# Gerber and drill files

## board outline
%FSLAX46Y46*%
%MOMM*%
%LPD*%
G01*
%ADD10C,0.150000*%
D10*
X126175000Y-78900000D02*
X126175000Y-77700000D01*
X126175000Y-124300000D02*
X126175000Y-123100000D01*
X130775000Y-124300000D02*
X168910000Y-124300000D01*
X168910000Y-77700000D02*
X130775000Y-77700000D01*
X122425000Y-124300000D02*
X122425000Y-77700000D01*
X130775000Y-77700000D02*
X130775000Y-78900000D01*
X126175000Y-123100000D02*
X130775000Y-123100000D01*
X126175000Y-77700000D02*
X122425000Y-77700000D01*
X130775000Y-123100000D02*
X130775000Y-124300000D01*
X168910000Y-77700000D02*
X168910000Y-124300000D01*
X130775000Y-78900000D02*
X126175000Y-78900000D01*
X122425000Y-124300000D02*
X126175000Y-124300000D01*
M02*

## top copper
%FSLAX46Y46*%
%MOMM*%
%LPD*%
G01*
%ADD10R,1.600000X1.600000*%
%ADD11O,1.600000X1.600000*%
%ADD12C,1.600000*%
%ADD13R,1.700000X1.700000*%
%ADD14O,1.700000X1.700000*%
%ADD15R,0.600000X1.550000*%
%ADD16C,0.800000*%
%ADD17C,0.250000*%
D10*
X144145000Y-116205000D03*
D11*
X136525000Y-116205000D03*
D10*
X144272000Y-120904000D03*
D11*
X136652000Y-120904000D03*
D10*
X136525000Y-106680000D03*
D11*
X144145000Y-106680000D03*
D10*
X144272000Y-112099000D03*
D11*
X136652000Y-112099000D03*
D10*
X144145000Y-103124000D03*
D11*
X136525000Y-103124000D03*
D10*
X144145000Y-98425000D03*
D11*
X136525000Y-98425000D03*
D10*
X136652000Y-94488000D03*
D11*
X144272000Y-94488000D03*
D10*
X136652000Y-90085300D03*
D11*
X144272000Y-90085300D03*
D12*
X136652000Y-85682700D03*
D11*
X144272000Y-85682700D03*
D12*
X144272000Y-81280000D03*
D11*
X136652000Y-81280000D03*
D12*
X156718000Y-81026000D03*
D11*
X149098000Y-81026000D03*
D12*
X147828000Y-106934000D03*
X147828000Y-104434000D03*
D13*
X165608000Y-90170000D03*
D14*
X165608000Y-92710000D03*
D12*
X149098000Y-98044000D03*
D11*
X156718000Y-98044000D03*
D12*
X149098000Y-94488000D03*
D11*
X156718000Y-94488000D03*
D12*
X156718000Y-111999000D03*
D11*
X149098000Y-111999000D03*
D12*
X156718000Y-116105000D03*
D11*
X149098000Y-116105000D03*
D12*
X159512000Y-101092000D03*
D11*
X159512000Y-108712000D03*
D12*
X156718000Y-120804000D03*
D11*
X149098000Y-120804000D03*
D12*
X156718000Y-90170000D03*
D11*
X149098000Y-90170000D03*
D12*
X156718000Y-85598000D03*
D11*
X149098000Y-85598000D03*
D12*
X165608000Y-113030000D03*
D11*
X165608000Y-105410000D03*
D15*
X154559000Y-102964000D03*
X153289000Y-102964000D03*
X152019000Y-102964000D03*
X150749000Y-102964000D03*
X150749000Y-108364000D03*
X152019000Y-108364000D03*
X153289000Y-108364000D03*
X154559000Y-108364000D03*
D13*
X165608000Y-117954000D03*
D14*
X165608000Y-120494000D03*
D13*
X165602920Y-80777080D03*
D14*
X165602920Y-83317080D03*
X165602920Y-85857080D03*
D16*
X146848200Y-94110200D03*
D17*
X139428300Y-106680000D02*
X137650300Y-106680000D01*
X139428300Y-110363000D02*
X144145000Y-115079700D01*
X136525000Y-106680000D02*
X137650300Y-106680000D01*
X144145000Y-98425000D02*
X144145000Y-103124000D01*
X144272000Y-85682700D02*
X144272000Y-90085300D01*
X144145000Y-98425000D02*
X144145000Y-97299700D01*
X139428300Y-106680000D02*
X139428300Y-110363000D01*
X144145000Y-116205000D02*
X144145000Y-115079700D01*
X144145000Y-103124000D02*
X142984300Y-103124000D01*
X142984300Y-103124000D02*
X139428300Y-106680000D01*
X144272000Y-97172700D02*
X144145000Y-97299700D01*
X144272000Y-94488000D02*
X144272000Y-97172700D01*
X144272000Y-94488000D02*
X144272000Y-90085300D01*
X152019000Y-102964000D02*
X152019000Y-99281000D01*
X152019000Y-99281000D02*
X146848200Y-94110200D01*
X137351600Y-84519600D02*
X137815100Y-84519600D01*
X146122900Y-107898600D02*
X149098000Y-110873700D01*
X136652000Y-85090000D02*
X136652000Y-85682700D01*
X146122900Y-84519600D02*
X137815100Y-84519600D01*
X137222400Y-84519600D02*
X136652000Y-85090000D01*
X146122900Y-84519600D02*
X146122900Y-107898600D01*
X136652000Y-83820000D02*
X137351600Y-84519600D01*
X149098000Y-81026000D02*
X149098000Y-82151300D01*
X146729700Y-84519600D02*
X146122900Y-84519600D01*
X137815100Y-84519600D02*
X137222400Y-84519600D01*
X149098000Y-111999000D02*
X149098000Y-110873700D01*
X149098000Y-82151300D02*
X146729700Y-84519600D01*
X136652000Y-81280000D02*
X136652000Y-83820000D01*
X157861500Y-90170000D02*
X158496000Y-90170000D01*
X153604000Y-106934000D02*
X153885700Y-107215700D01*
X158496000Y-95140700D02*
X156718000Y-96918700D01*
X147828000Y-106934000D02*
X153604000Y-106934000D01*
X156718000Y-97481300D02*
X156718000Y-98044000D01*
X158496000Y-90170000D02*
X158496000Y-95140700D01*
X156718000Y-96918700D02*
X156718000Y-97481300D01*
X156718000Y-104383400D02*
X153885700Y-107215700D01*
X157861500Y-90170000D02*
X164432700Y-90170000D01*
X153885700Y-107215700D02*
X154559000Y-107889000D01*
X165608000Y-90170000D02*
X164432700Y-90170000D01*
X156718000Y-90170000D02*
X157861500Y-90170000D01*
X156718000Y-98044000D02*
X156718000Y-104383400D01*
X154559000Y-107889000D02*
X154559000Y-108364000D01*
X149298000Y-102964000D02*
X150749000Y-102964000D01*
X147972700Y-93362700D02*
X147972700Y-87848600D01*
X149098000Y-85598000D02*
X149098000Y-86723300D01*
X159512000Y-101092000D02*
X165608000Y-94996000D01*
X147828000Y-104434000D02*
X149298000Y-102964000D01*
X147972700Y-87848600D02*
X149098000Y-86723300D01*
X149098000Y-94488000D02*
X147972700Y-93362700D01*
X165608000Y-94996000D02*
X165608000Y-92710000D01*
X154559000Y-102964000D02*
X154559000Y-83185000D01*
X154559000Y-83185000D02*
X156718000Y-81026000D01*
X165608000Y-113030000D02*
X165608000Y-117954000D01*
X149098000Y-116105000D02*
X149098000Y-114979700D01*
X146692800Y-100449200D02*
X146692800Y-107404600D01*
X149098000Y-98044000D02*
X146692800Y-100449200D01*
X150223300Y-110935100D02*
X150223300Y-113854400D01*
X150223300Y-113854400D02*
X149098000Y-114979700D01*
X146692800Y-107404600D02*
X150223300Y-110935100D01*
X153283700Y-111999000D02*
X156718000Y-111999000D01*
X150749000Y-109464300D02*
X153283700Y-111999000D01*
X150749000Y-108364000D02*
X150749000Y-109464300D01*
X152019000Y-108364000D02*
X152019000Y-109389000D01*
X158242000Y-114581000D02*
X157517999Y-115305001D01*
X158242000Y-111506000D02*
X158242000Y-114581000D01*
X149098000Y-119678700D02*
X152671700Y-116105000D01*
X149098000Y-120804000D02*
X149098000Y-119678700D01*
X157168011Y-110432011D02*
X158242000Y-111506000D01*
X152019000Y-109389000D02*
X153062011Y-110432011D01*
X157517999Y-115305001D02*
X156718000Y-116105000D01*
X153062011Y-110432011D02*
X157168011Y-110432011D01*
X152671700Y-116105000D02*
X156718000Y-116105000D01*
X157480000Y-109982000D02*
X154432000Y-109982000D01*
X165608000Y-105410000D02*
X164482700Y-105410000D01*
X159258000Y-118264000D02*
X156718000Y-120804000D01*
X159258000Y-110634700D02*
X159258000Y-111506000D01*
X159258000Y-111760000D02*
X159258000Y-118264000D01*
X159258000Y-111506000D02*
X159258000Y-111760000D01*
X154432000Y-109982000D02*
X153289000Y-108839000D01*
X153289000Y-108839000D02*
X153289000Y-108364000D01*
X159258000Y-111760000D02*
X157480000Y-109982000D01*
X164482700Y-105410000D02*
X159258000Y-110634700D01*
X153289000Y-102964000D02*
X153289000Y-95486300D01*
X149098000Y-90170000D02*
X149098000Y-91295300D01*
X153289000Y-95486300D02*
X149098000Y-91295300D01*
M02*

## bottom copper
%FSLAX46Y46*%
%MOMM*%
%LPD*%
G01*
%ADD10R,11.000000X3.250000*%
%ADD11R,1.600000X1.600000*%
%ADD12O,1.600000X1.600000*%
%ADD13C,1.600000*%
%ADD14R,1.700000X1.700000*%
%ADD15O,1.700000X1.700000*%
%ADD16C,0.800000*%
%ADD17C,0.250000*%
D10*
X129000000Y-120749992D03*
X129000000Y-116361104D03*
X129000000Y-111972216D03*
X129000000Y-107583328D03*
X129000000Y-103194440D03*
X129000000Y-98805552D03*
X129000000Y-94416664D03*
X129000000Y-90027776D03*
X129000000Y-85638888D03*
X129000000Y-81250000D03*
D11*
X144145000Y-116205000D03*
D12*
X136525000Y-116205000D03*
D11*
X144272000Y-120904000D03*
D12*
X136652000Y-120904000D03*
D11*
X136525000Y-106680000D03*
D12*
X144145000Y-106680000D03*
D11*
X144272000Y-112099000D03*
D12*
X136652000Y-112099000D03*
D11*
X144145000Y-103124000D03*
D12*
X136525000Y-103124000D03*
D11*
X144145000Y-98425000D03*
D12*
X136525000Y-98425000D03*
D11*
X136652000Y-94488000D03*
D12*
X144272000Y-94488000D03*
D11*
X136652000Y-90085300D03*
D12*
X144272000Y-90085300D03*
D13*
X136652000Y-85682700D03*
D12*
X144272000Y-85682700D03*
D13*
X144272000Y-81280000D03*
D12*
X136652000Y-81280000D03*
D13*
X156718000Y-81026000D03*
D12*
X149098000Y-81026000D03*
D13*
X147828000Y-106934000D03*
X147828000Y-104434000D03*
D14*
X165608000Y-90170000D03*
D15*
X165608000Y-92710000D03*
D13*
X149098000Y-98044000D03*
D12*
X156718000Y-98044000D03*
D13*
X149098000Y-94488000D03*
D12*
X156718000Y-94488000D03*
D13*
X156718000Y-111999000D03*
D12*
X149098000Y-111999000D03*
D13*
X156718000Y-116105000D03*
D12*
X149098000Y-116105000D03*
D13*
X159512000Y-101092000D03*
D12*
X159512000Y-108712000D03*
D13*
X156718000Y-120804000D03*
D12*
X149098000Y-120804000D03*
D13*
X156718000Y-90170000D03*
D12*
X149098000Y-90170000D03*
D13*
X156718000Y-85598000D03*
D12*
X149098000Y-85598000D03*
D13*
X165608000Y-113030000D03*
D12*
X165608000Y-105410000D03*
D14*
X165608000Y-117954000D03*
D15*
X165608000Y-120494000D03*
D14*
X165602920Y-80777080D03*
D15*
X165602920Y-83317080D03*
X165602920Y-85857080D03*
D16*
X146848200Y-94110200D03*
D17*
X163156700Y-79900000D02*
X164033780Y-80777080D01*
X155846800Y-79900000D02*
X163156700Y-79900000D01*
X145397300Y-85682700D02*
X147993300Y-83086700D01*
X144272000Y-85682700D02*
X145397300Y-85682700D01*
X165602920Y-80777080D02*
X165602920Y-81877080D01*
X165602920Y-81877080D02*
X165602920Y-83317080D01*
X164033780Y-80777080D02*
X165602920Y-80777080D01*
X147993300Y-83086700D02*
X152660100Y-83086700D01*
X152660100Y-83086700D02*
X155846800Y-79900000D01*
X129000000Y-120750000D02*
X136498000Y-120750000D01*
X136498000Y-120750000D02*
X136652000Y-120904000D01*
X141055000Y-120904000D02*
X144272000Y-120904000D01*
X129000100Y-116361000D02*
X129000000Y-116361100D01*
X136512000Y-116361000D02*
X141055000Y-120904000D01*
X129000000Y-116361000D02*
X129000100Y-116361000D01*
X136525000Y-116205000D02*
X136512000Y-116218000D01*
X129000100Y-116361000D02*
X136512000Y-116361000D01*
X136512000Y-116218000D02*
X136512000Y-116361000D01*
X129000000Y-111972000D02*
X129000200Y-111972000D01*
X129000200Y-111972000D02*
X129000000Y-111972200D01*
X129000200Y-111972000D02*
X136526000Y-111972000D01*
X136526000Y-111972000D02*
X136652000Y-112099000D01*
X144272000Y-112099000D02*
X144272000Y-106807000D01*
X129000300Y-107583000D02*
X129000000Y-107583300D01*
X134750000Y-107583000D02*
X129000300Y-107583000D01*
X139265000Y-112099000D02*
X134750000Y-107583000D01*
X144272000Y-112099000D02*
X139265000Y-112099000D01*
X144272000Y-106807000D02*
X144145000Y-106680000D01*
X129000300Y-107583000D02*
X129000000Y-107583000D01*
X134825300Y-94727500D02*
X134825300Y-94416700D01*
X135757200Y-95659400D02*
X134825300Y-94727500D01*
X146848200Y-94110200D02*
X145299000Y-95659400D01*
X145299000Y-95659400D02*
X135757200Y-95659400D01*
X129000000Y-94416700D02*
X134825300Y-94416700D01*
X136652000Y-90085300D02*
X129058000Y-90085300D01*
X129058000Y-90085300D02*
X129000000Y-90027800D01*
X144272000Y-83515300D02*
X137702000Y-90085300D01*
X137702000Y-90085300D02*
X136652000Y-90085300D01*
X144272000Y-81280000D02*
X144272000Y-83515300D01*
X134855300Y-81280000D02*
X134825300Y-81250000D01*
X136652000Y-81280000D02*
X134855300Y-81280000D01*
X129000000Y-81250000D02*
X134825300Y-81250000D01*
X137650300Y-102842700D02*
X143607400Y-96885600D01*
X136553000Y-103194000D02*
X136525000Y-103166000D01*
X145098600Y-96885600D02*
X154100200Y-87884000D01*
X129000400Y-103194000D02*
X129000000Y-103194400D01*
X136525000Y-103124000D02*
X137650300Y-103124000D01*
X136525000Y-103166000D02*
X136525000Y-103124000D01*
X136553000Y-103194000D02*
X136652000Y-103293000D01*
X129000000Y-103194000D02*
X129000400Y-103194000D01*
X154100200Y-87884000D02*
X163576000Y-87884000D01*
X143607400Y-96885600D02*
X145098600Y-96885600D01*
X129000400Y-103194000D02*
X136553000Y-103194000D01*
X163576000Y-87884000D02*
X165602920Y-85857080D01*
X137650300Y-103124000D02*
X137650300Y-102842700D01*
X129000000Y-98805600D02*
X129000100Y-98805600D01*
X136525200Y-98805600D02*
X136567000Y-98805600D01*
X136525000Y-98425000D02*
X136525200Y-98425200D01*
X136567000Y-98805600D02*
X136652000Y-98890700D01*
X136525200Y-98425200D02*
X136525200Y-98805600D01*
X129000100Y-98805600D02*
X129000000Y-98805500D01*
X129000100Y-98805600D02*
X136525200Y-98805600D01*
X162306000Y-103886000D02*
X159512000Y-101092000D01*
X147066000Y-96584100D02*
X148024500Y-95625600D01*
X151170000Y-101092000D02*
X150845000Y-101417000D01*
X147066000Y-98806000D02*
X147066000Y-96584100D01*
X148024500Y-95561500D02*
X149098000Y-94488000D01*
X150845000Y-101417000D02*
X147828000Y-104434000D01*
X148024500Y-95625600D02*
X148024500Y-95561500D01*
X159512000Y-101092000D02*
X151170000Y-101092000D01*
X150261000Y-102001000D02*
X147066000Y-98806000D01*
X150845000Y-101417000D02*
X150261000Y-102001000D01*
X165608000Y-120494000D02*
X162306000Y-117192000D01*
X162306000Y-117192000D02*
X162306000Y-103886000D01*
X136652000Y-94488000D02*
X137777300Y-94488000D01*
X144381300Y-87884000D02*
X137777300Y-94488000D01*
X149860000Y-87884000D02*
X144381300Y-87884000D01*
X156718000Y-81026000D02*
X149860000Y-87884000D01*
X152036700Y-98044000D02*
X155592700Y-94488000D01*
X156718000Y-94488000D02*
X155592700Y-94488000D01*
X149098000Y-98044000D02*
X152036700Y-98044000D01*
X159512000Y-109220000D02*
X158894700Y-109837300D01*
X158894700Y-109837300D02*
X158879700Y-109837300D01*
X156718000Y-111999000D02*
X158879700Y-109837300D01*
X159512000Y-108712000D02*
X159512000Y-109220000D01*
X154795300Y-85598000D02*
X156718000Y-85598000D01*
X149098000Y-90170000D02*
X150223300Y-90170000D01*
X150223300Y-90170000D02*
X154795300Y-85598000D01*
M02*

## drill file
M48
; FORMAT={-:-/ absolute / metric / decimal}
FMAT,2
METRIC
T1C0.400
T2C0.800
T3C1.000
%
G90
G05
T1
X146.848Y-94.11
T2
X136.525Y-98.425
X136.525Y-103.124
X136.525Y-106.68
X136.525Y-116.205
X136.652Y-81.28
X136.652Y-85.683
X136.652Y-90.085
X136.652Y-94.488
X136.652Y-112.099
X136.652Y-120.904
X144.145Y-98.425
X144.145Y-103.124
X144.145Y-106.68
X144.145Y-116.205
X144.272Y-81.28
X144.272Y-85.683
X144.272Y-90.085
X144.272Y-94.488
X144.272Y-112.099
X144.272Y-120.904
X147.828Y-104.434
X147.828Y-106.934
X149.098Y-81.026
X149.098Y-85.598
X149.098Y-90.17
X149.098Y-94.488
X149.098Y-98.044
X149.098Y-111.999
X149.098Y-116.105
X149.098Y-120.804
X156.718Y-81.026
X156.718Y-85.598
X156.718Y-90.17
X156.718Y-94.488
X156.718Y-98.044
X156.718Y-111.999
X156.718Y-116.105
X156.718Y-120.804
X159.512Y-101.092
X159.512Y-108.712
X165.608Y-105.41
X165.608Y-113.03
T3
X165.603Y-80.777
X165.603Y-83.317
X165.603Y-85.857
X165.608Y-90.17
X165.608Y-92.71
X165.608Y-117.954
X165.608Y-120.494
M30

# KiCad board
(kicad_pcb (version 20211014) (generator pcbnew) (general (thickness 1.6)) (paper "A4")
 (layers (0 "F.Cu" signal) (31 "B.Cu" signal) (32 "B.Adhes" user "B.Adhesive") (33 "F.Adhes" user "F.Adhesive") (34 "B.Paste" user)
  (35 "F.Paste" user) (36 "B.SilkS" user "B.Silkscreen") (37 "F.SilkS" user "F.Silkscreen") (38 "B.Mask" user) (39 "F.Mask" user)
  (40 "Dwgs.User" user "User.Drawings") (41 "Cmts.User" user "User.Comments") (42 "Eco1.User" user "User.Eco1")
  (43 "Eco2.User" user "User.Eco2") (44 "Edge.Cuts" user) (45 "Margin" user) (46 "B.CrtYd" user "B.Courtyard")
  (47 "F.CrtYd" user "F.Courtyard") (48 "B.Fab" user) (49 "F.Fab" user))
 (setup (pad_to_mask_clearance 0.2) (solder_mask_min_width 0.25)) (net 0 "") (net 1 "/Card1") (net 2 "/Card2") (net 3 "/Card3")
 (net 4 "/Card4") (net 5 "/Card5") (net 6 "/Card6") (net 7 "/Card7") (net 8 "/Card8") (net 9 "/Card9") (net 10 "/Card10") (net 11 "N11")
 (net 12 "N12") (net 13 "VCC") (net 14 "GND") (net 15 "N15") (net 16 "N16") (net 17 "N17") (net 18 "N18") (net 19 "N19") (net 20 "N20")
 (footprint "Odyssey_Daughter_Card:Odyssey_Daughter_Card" (layer "F.Cu") (at 129 101)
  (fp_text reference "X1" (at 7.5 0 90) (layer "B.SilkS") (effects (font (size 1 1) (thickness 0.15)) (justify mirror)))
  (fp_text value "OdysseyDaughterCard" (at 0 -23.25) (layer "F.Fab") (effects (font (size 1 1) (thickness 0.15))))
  (pad "1" smd rect locked (at 0 19.749992) (size 11 3.25) (layers "B.Cu" "B.Mask") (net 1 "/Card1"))
  (pad "2" smd rect locked (at 0 15.361104) (size 11 3.25) (layers "B.Cu" "B.Mask") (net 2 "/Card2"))
  (pad "3" smd rect locked (at 0 10.972216) (size 11 3.25) (layers "B.Cu" "B.Mask") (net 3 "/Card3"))
  (pad "4" smd rect locked (at 0 6.583328) (size 11 3.25) (layers "B.Cu" "B.Mask") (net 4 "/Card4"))
  (pad "5" smd rect locked (at 0 2.19444) (size 11 3.25) (layers "B.Cu" "B.Mask") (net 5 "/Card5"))
  (pad "6" smd rect locked (at 0 -2.194448) (size 11 3.25) (layers "B.Cu" "B.Mask") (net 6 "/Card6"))
  (pad "7" smd rect locked (at 0 -6.583336) (size 11 3.25) (layers "B.Cu" "B.Mask") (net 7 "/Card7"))
  (pad "8" smd rect locked (at 0 -10.972224) (size 11 3.25) (layers "B.Cu" "B.Mask") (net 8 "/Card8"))
  (pad "9" smd rect locked (at 0 -15.361112) (size 11 3.25) (layers "B.Cu" "B.Mask") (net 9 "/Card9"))
  (pad "10" smd rect locked (at 0 -19.75) (size 11 3.25) (layers "B.Cu" "B.Mask") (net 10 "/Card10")))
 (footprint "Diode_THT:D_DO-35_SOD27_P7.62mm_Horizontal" (layer "F.Cu") (at 144.145 116.205 180)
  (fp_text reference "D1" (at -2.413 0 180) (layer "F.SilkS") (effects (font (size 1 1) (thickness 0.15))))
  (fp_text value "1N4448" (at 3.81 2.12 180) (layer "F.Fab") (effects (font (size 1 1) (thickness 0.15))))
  (pad "1" thru_hole rect locked (at 0 0 180) (size 1.6 1.6) (drill 0.8) (layers *.Cu *.Mask) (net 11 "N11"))
  (pad "2" thru_hole oval locked (at 7.62 0 180) (size 1.6 1.6) (drill 0.8) (layers *.Cu *.Mask) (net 2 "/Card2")))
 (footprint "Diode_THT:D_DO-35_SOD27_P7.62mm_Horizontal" (layer "F.Cu") (at 144.272 120.904 180)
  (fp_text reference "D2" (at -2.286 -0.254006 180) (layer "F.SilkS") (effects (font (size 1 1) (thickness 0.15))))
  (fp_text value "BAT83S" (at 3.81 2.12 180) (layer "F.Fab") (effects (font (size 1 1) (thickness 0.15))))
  (pad "1" thru_hole rect locked (at 0 0 180) (size 1.6 1.6) (drill 0.8) (layers *.Cu *.Mask) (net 2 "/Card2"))
  (pad "2" thru_hole oval locked (at 7.62 0 180) (size 1.6 1.6) (drill 0.8) (layers *.Cu *.Mask) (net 1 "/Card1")))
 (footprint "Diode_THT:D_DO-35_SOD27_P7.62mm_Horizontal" (layer "F.Cu") (at 136.525 106.68)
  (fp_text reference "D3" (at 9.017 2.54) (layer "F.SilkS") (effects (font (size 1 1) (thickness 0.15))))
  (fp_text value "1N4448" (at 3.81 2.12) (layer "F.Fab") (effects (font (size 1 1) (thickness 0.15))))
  (pad "1" thru_hole rect locked (at 0 0) (size 1.6 1.6) (drill 0.8) (layers *.Cu *.Mask) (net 11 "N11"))
  (pad "2" thru_hole oval locked (at 7.62 0) (size 1.6 1.6) (drill 0.8) (layers *.Cu *.Mask) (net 4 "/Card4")))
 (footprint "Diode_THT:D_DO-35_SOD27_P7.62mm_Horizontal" (layer "F.Cu") (at 144.272 112.099 180)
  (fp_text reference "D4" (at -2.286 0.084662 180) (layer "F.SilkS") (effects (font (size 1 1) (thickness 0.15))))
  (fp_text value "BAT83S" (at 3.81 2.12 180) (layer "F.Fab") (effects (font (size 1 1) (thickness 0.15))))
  (pad "1" thru_hole rect locked (at 0 0 180) (size 1.6 1.6) (drill 0.8) (layers *.Cu *.Mask) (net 4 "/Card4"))
  (pad "2" thru_hole oval locked (at 7.62 0 180) (size 1.6 1.6) (drill 0.8) (layers *.Cu *.Mask) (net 3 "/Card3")))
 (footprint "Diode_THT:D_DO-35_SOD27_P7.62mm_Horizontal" (layer "F.Cu") (at 144.145 103.124 180)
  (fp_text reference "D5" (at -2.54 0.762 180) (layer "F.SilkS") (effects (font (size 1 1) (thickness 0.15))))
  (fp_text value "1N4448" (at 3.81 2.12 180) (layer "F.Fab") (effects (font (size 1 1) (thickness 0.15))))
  (pad "1" thru_hole rect locked (at 0 0 180) (size 1.6 1.6) (drill 0.8) (layers *.Cu *.Mask) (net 11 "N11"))
  (pad "2" thru_hole oval locked (at 7.62 0 180) (size 1.6 1.6) (drill 0.8) (layers *.Cu *.Mask) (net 5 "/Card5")))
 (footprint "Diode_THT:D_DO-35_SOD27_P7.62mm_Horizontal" (layer "F.Cu") (at 144.145 98.425 180)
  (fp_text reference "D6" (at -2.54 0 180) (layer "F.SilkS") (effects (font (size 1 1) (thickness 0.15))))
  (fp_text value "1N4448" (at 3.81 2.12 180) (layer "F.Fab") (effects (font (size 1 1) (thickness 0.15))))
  (pad "1" thru_hole rect locked (at 0 0 180) (size 1.6 1.6) (drill 0.8) (layers *.Cu *.Mask) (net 11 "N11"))
  (pad "2" thru_hole oval locked (at 7.62 0 180) (size 1.6 1.6) (drill 0.8) (layers *.Cu *.Mask) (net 6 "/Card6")))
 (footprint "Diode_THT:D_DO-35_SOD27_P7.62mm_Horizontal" (layer "F.Cu") (at 136.652 94.488)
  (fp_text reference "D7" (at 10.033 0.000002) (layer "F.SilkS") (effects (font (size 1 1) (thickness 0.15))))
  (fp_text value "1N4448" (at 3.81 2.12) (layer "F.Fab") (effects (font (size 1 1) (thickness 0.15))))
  (pad "1" thru_hole rect locked (at 0 0) (size 1.6 1.6) (drill 0.8) (layers *.Cu *.Mask) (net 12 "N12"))
  (pad "2" thru_hole oval locked (at 7.62 0) (size 1.6 1.6) (drill 0.8) (layers *.Cu *.Mask) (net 11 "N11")))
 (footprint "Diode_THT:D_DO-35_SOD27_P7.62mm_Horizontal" (layer "F.Cu") (at 136.652 90.0853)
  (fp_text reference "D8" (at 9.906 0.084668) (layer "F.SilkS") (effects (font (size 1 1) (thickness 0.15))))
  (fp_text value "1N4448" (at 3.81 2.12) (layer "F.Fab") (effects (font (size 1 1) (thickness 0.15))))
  (pad "1" thru_hole rect locked (at 0 0) (size 1.6 1.6) (drill 0.8) (layers *.Cu *.Mask) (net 8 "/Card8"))
  (pad "2" thru_hole oval locked (at 7.62 0) (size 1.6 1.6) (drill 0.8) (layers *.Cu *.Mask) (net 11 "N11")))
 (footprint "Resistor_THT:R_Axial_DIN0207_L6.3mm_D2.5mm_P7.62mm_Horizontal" (layer "F.Cu") (at 136.652 85.6827)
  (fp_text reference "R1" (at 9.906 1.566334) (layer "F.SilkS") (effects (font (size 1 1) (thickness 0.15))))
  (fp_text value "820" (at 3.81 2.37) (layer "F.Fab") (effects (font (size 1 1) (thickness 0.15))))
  (pad "1" thru_hole circle locked (at 0 0) (size 1.6 1.6) (drill 0.8) (layers *.Cu *.Mask) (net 10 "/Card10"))
  (pad "2" thru_hole oval locked (at 7.62 0) (size 1.6 1.6) (drill 0.8) (layers *.Cu *.Mask) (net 11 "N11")))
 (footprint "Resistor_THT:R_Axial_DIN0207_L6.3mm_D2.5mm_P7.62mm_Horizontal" (layer "F.Cu") (at 144.272 81.28 180)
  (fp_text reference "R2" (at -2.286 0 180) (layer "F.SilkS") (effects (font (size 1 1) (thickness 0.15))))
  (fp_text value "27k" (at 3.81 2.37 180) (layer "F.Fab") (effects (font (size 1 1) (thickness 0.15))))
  (pad "1" thru_hole circle locked (at 0 0 180) (size 1.6 1.6) (drill 0.8) (layers *.Cu *.Mask) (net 8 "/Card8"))
  (pad "2" thru_hole oval locked (at 7.62 0 180) (size 1.6 1.6) (drill 0.8) (layers *.Cu *.Mask) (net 10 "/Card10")))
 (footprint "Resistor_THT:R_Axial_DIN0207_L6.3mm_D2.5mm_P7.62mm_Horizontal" (layer "F.Cu") (at 156.718 81.026 180)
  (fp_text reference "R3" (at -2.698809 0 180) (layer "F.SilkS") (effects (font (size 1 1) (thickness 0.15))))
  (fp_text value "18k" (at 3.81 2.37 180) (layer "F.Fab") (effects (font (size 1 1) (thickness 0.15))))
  (pad "1" thru_hole circle locked (at 0 0 180) (size 1.6 1.6) (drill 0.8) (layers *.Cu *.Mask) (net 12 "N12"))
  (pad "2" thru_hole oval locked (at 7.62 0 180) (size 1.6 1.6) (drill 0.8) (layers *.Cu *.Mask) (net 10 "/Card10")))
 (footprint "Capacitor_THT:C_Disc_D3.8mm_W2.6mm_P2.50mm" (layer "F.Cu") (at 147.828 106.934 90)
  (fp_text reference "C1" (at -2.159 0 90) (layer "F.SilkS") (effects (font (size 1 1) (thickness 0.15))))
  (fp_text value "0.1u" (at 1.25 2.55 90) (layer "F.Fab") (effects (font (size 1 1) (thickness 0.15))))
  (pad "1" thru_hole circle locked (at 0 0 90) (size 1.6 1.6) (drill 0.8) (layers *.Cu *.Mask) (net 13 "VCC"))
  (pad "2" thru_hole circle locked (at 2.5 0 90) (size 1.6 1.6) (drill 0.8) (layers *.Cu *.Mask) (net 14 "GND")))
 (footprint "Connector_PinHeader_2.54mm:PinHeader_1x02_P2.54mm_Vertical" (layer "F.Cu") (at 165.608 90.17)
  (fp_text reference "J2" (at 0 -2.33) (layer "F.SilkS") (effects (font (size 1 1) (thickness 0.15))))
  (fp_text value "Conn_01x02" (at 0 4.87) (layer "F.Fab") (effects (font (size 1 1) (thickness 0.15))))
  (pad "1" thru_hole rect locked (at 0 0) (size 1.7 1.7) (drill 1) (layers *.Cu *.Mask) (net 13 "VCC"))
  (pad "2" thru_hole oval locked (at 0 2.54) (size 1.7 1.7) (drill 1) (layers *.Cu *.Mask) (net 14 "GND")))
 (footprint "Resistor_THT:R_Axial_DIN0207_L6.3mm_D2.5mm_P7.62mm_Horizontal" (layer "F.Cu") (at 149.098 98.044)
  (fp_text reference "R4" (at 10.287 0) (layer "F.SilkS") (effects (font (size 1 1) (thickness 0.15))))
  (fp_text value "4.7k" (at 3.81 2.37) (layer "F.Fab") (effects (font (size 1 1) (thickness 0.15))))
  (pad "1" thru_hole circle locked (at 0 0) (size 1.6 1.6) (drill 0.8) (layers *.Cu *.Mask) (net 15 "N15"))
  (pad "2" thru_hole oval locked (at 7.62 0) (size 1.6 1.6) (drill 0.8) (layers *.Cu *.Mask) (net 13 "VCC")))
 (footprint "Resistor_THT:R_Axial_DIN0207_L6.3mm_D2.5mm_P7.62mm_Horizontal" (layer "F.Cu") (at 149.098 94.488)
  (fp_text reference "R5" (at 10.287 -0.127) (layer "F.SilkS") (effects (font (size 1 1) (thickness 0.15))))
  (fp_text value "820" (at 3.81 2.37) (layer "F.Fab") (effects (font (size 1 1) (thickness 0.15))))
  (pad "1" thru_hole circle locked (at 0 0) (size 1.6 1.6) (drill 0.8) (layers *.Cu *.Mask) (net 14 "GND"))
  (pad "2" thru_hole oval locked (at 7.62 0) (size 1.6 1.6) (drill 0.8) (layers *.Cu *.Mask) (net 15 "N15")))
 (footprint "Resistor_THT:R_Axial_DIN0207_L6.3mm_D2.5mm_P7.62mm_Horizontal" (layer "F.Cu") (at 156.718 111.999 180)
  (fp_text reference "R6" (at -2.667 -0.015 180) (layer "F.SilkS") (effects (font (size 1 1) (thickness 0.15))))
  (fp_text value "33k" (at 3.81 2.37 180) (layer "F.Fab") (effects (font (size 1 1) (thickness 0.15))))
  (pad "1" thru_hole circle locked (at 0 0 180) (size 1.6 1.6) (drill 0.8) (layers *.Cu *.Mask) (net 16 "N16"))
  (pad "2" thru_hole oval locked (at 7.62 0 180) (size 1.6 1.6) (drill 0.8) (layers *.Cu *.Mask) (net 10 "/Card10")))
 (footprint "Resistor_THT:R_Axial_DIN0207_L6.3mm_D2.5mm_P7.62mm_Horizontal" (layer "F.Cu") (at 156.718 116.105 180)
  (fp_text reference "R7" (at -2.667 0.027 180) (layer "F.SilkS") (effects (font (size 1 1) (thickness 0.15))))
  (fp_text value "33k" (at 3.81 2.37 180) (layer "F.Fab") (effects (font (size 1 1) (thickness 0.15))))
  (pad "1" thru_hole circle locked (at 0 0 180) (size 1.6 1.6) (drill 0.8) (layers *.Cu *.Mask) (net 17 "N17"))
  (pad "2" thru_hole oval locked (at 7.62 0 180) (size 1.6 1.6) (drill 0.8) (layers *.Cu *.Mask) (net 15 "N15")))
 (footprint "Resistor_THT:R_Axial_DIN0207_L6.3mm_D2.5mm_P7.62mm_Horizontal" (layer "F.Cu") (at 159.512 101.092 -90)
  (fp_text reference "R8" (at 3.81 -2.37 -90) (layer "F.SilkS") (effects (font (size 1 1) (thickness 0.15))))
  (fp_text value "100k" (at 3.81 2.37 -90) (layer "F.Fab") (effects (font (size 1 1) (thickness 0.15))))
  (pad "1" thru_hole circle locked (at 0 0 270) (size 1.6 1.6) (drill 0.8) (layers *.Cu *.Mask) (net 14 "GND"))
  (pad "2" thru_hole oval locked (at 7.62 0 270) (size 1.6 1.6) (drill 0.8) (layers *.Cu *.Mask) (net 16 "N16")))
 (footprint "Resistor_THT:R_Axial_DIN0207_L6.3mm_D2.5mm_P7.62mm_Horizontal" (layer "F.Cu") (at 156.718 120.804 180)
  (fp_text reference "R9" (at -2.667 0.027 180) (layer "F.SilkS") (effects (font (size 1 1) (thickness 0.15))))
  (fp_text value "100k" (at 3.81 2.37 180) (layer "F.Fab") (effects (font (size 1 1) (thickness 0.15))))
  (pad "1" thru_hole circle locked (at 0 0 180) (size 1.6 1.6) (drill 0.8) (layers *.Cu *.Mask) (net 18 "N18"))
  (pad "2" thru_hole oval locked (at 7.62 0 180) (size 1.6 1.6) (drill 0.8) (layers *.Cu *.Mask) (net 17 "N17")))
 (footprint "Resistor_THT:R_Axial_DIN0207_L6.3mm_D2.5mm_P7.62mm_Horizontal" (layer "F.Cu") (at 156.718 90.17 180)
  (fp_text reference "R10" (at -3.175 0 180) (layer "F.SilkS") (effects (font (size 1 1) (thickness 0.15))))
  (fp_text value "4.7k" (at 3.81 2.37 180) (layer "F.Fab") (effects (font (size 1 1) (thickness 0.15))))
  (pad "1" thru_hole circle locked (at 0 0 180) (size 1.6 1.6) (drill 0.8) (layers *.Cu *.Mask) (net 13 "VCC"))
  (pad "2" thru_hole oval locked (at 7.62 0 180) (size 1.6 1.6) (drill 0.8) (layers *.Cu *.Mask) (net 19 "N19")))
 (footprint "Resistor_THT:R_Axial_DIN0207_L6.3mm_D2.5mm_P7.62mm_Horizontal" (layer "F.Cu") (at 156.718 85.598 180)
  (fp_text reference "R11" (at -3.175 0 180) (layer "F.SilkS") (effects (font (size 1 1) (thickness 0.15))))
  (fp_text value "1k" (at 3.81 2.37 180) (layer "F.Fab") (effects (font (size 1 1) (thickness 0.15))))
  (pad "1" thru_hole circle locked (at 0 0 180) (size 1.6 1.6) (drill 0.8) (layers *.Cu *.Mask) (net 19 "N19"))
  (pad "2" thru_hole oval locked (at 7.62 0 180) (size 1.6 1.6) (drill 0.8) (layers *.Cu *.Mask) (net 14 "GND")))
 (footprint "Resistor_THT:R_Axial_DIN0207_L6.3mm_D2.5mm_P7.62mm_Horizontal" (layer "F.Cu") (at 165.608 113.03 90)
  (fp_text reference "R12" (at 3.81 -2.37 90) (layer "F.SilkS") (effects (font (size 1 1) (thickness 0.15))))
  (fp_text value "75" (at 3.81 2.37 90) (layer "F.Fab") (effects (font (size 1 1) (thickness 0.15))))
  (pad "1" thru_hole circle locked (at 0 0 90) (size 1.6 1.6) (drill 0.8) (layers *.Cu *.Mask) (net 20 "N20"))
  (pad "2" thru_hole oval locked (at 7.62 0 90) (size 1.6 1.6) (drill 0.8) (layers *.Cu *.Mask) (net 18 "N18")))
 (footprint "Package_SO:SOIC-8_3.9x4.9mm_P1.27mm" (layer "F.Cu") (at 152.654 105.664 -90)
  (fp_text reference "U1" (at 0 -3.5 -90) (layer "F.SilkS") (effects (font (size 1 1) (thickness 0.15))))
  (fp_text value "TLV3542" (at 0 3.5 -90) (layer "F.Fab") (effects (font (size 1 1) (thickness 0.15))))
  (pad "1" smd rect locked (at -2.7 -1.905 270) (size 1.55 0.6) (layers "F.Cu" "F.Paste" "F.Mask") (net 12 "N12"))
  (pad "2" smd rect locked (at -2.7 -0.635 270) (size 1.55 0.6) (layers "F.Cu" "F.Paste" "F.Mask") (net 19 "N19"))
  (pad "3" smd rect locked (at -2.7 0.635 270) (size 1.55 0.6) (layers "F.Cu" "F.Paste" "F.Mask") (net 7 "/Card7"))
  (pad "4" smd rect locked (at -2.7 1.905 270) (size 1.55 0.6) (layers "F.Cu" "F.Paste" "F.Mask") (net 14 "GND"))
  (pad "5" smd rect locked (at 2.7 1.905 270) (size 1.55 0.6) (layers "F.Cu" "F.Paste" "F.Mask") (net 16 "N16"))
  (pad "6" smd rect locked (at 2.7 0.635 270) (size 1.55 0.6) (layers "F.Cu" "F.Paste" "F.Mask") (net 17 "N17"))
  (pad "7" smd rect locked (at 2.7 -0.635 270) (size 1.55 0.6) (layers "F.Cu" "F.Paste" "F.Mask") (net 18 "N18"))
  (pad "8" smd rect locked (at 2.7 -1.905 270) (size 1.55 0.6) (layers "F.Cu" "F.Paste" "F.Mask") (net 13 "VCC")))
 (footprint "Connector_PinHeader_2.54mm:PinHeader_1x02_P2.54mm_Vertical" (layer "F.Cu") (at 165.608 117.954)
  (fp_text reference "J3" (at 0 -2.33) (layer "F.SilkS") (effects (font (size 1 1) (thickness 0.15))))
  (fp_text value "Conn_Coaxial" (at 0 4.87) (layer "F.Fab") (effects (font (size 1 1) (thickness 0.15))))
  (pad "1" thru_hole rect locked (at 0 0) (size 1.7 1.7) (drill 1) (layers *.Cu *.Mask) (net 20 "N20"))
  (pad "2" thru_hole oval locked (at 0 2.54) (size 1.7 1.7) (drill 1) (layers *.Cu *.Mask) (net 14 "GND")))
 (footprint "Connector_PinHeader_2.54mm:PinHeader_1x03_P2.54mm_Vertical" (layer "F.Cu") (at 165.60292 80.77708)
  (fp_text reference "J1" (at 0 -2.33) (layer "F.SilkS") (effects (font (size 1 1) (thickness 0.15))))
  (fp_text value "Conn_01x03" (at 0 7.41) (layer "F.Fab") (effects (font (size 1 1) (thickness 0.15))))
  (pad "1" thru_hole rect locked (at 0 0) (size 1.7 1.7) (drill 1) (layers *.Cu *.Mask) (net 11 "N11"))
  (pad "2" thru_hole oval locked (at 0 2.54) (size 1.7 1.7) (drill 1) (layers *.Cu *.Mask) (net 11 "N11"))
  (pad "3" thru_hole oval locked (at 0 5.08) (size 1.7 1.7) (drill 1) (layers *.Cu *.Mask) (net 5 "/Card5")))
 (gr_line (start 126.175 78.9) (end 126.175 77.7) (layer "Edge.Cuts") (width 0.15))
 (gr_line (start 126.175 124.3) (end 126.175 123.1) (layer "Edge.Cuts") (width 0.15))
 (gr_line (start 130.775 124.3) (end 168.91 124.3) (layer "Edge.Cuts") (width 0.15))
 (gr_line (start 168.91 77.7) (end 130.775 77.7) (layer "Edge.Cuts") (width 0.15))
 (gr_line (start 122.425 124.3) (end 122.425 77.7) (layer "Edge.Cuts") (width 0.15))
 (gr_line (start 130.775 77.7) (end 130.775 78.9) (layer "Edge.Cuts") (width 0.15))
 (gr_line (start 126.175 123.1) (end 130.775 123.1) (layer "Edge.Cuts") (width 0.15))
 (gr_line (start 126.175 77.7) (end 122.425 77.7) (layer "Edge.Cuts") (width 0.15))
 (gr_line (start 130.775 123.1) (end 130.775 124.3) (layer "Edge.Cuts") (width 0.15))
 (gr_line (start 168.91 77.7) (end 168.91 124.3) (layer "Edge.Cuts") (width 0.15))
 (gr_line (start 130.775 78.9) (end 126.175 78.9) (layer "Edge.Cuts") (width 0.15))
 (gr_line (start 122.425 124.3) (end 126.175 124.3) (layer "Edge.Cuts") (width 0.15))
 (segment (start 139.4283 106.68) (end 137.6503 106.68) (width 0.25) (layer "F.Cu") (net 11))
 (segment (start 139.4283 110.363) (end 144.145 115.0797) (width 0.25) (layer "F.Cu") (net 11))
 (segment (start 136.525 106.68) (end 137.6503 106.68) (width 0.25) (layer "F.Cu") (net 11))
 (segment (start 144.145 98.425) (end 144.145 103.124) (width 0.25) (layer "F.Cu") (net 11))
 (segment (start 144.272 85.6827) (end 144.272 90.0853) (width 0.25) (layer "F.Cu") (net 11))
 (segment (start 144.145 98.425) (end 144.145 97.2997) (width 0.25) (layer "F.Cu") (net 11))
 (segment (start 139.4283 106.68) (end 139.4283 110.363) (width 0.25) (layer "F.Cu") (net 11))
 (segment (start 144.145 116.205) (end 144.145 115.0797) (width 0.25) (layer "F.Cu") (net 11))
 (segment (start 144.145 103.124) (end 142.9843 103.124) (width 0.25) (layer "F.Cu") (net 11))
 (segment (start 142.9843 103.124) (end 139.4283 106.68) (width 0.25) (layer "F.Cu") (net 11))
 (segment (start 144.272 97.1727) (end 144.145 97.2997) (width 0.25) (layer "F.Cu") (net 11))
 (segment (start 144.272 94.488) (end 144.272 97.1727) (width 0.25) (layer "F.Cu") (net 11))
 (segment (start 144.272 94.488) (end 144.272 90.0853) (width 0.25) (layer "F.Cu") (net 11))
 (segment (start 163.1567 79.9) (end 164.03378 80.77708) (width 0.25) (layer "B.Cu") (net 11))
 (segment (start 155.8468 79.9) (end 163.1567 79.9) (width 0.25) (layer "B.Cu") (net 11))
 (segment (start 145.3973 85.6827) (end 147.9933 83.0867) (width 0.25) (layer "B.Cu") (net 11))
 (segment (start 144.272 85.6827) (end 145.3973 85.6827) (width 0.25) (layer "B.Cu") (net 11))
 (segment (start 165.60292 80.77708) (end 165.60292 81.87708) (width 0.25) (layer "B.Cu") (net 11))
 (segment (start 165.60292 81.87708) (end 165.60292 83.31708) (width 0.25) (layer "B.Cu") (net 11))
 (segment (start 164.03378 80.77708) (end 165.60292 80.77708) (width 0.25) (layer "B.Cu") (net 11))
 (segment (start 147.9933 83.0867) (end 152.6601 83.0867) (width 0.25) (layer "B.Cu") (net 11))
 (segment (start 152.6601 83.0867) (end 155.8468 79.9) (width 0.25) (layer "B.Cu") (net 11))
 (segment (start 129 120.75) (end 136.498 120.75) (width 0.25) (layer "B.Cu") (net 1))
 (segment (start 136.498 120.75) (end 136.652 120.904) (width 0.25) (layer "B.Cu") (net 1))
 (segment (start 141.055 120.904) (end 144.272 120.904) (width 0.25) (layer "B.Cu") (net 2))
 (segment (start 129.0001 116.361) (end 129 116.3611) (width 0.25) (layer "B.Cu") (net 2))
 (segment (start 136.512 116.361) (end 141.055 120.904) (width 0.25) (layer "B.Cu") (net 2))
 (segment (start 129 116.361) (end 129.0001 116.361) (width 0.25) (layer "B.Cu") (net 2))
 (segment (start 136.525 116.205) (end 136.512 116.218) (width 0.25) (layer "B.Cu") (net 2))
 (segment (start 129.0001 116.361) (end 136.512 116.361) (width 0.25) (layer "B.Cu") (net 2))
 (segment (start 136.512 116.218) (end 136.512 116.361) (width 0.25) (layer "B.Cu") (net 2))
 (segment (start 129 111.972) (end 129.0002 111.972) (width 0.25) (layer "B.Cu") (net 3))
 (segment (start 129.0002 111.972) (end 129 111.9722) (width 0.25) (layer "B.Cu") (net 3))
 (segment (start 129.0002 111.972) (end 136.526 111.972) (width 0.25) (layer "B.Cu") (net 3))
 (segment (start 136.526 111.972) (end 136.652 112.099) (width 0.25) (layer "B.Cu") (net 3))
 (segment (start 144.272 112.099) (end 144.272 106.807) (width 0.25) (layer "B.Cu") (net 4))
 (segment (start 129.0003 107.583) (end 129 107.5833) (width 0.25) (layer "B.Cu") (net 4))
 (segment (start 134.75 107.583) (end 129.0003 107.583) (width 0.25) (layer "B.Cu") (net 4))
 (segment (start 139.265 112.099) (end 134.75 107.583) (width 0.25) (layer "B.Cu") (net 4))
 (segment (start 144.272 112.099) (end 139.265 112.099) (width 0.25) (layer "B.Cu") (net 4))
 (segment (start 144.272 106.807) (end 144.145 106.68) (width 0.25) (layer "B.Cu") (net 4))
 (segment (start 129.0003 107.583) (end 129 107.583) (width 0.25) (layer "B.Cu") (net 4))
 (segment (start 152.019 102.964) (end 152.019 99.281) (width 0.25) (layer "F.Cu") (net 7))
 (segment (start 152.019 99.281) (end 146.8482 94.1102) (width 0.25) (layer "F.Cu") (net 7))
 (via (at 146.8482 94.1102) (size 0.8) (drill 0.4) (layers "F.Cu" "B.Cu") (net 7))
 (segment (start 134.8253 94.7275) (end 134.8253 94.4167) (width 0.25) (layer "B.Cu") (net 7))
 (segment (start 135.7572 95.6594) (end 134.8253 94.7275) (width 0.25) (layer "B.Cu") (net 7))
 (segment (start 146.8482 94.1102) (end 145.299 95.6594) (width 0.25) (layer "B.Cu") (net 7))
 (segment (start 145.299 95.6594) (end 135.7572 95.6594) (width 0.25) (layer "B.Cu") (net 7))
 (segment (start 129 94.4167) (end 134.8253 94.4167) (width 0.25) (layer "B.Cu") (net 7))
 (segment (start 136.652 90.0853) (end 129.058 90.0853) (width 0.25) (layer "B.Cu") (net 8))
 (segment (start 129.058 90.0853) (end 129 90.0278) (width 0.25) (layer "B.Cu") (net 8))
 (segment (start 144.272 83.5153) (end 137.702 90.0853) (width 0.25) (layer "B.Cu") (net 8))
 (segment (start 137.702 90.0853) (end 136.652 90.0853) (width 0.25) (layer "B.Cu") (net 8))
 (segment (start 144.272 81.28) (end 144.272 83.5153) (width 0.25) (layer "B.Cu") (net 8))
 (segment (start 137.3516 84.5196) (end 137.8151 84.5196) (width 0.25) (layer "F.Cu") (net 10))
 (segment (start 146.1229 107.8986) (end 149.098 110.8737) (width 0.25) (layer "F.Cu") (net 10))
 (segment (start 136.652 85.09) (end 136.652 85.6827) (width 0.25) (layer "F.Cu") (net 10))
 (segment (start 146.1229 84.5196) (end 137.8151 84.5196) (width 0.25) (layer "F.Cu") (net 10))
 (segment (start 137.2224 84.5196) (end 136.652 85.09) (width 0.25) (layer "F.Cu") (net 10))
 (segment (start 146.1229 84.5196) (end 146.1229 107.8986) (width 0.25) (layer "F.Cu") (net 10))
 (segment (start 136.652 83.82) (end 137.3516 84.5196) (width 0.25) (layer "F.Cu") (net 10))
 (segment (start 149.098 81.026) (end 149.098 82.1513) (width 0.25) (layer "F.Cu") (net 10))
 (segment (start 146.7297 84.5196) (end 146.1229 84.5196) (width 0.25) (layer "F.Cu") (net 10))
 (segment (start 137.8151 84.5196) (end 137.2224 84.5196) (width 0.25) (layer "F.Cu") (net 10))
 (segment (start 149.098 111.999) (end 149.098 110.8737) (width 0.25) (layer "F.Cu") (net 10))
 (segment (start 149.098 82.1513) (end 146.7297 84.5196) (width 0.25) (layer "F.Cu") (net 10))
 (segment (start 136.652 81.28) (end 136.652 83.82) (width 0.25) (layer "F.Cu") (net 10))
 (segment (start 134.8553 81.28) (end 134.8253 81.25) (width 0.25) (layer "B.Cu") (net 10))
 (segment (start 136.652 81.28) (end 134.8553 81.28) (width 0.25) (layer "B.Cu") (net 10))
 (segment (start 129 81.25) (end 134.8253 81.25) (width 0.25) (layer "B.Cu") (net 10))
 (segment (start 137.6503 102.8427) (end 143.6074 96.8856) (width 0.25) (layer "B.Cu") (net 5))
 (segment (start 136.553 103.194) (end 136.525 103.166) (width 0.25) (layer "B.Cu") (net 5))
 (segment (start 145.0986 96.8856) (end 154.1002 87.884) (width 0.25) (layer "B.Cu") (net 5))
 (segment (start 129.0004 103.194) (end 129 103.1944) (width 0.25) (layer "B.Cu") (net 5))
 (segment (start 136.525 103.124) (end 137.6503 103.124) (width 0.25) (layer "B.Cu") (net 5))
 (segment (start 136.525 103.166) (end 136.525 103.124) (width 0.25) (layer "B.Cu") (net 5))
 (segment (start 136.553 103.194) (end 136.652 103.293) (width 0.25) (layer "B.Cu") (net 5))
 (segment (start 129 103.194) (end 129.0004 103.194) (width 0.25) (layer "B.Cu") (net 5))
 (segment (start 154.1002 87.884) (end 163.576 87.884) (width 0.25) (layer "B.Cu") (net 5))
 (segment (start 143.6074 96.8856) (end 145.0986 96.8856) (width 0.25) (layer "B.Cu") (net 5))
 (segment (start 129.0004 103.194) (end 136.553 103.194) (width 0.25) (layer "B.Cu") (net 5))
 (segment (start 163.576 87.884) (end 165.60292 85.85708) (width 0.25) (layer "B.Cu") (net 5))
 (segment (start 137.6503 103.124) (end 137.6503 102.8427) (width 0.25) (layer "B.Cu") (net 5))
 (segment (start 129 98.8056) (end 129.0001 98.8056) (width 0.25) (layer "B.Cu") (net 6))
 (segment (start 136.5252 98.8056) (end 136.567 98.8056) (width 0.25) (layer "B.Cu") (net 6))
 (segment (start 136.525 98.425) (end 136.5252 98.4252) (width 0.25) (layer "B.Cu") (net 6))
 (segment (start 136.567 98.8056) (end 136.652 98.8907) (width 0.25) (layer "B.Cu") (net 6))
 (segment (start 136.5252 98.4252) (end 136.5252 98.8056) (width 0.25) (layer "B.Cu") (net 6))
 (segment (start 129.0001 98.8056) (end 129 98.8055) (width 0.25) (layer "B.Cu") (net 6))
 (segment (start 129.0001 98.8056) (end 136.5252 98.8056) (width 0.25) (layer "B.Cu") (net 6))
 (segment (start 157.8615 90.17) (end 158.496 90.17) (width 0.25) (layer "F.Cu") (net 13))
 (segment (start 153.604 106.934) (end 153.8857 107.2157) (width 0.25) (layer "F.Cu") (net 13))
 (segment (start 158.496 95.1407) (end 156.718 96.9187) (width 0.25) (layer "F.Cu") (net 13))
 (segment (start 147.828 106.934) (end 153.604 106.934) (width 0.25) (layer "F.Cu") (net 13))
 (segment (start 156.718 97.4813) (end 156.718 98.044) (width 0.25) (layer "F.Cu") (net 13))
 (segment (start 158.496 90.17) (end 158.496 95.1407) (width 0.25) (layer "F.Cu") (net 13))
 (segment (start 156.718 96.9187) (end 156.718 97.4813) (width 0.25) (layer "F.Cu") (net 13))
 (segment (start 156.718 104.3834) (end 153.8857 107.2157) (width 0.25) (layer "F.Cu") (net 13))
 (segment (start 157.8615 90.17) (end 164.4327 90.17) (width 0.25) (layer "F.Cu") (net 13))
 (segment (start 153.8857 107.2157) (end 154.559 107.889) (width 0.25) (layer "F.Cu") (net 13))
 (segment (start 165.608 90.17) (end 164.4327 90.17) (width 0.25) (layer "F.Cu") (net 13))
 (segment (start 156.718 90.17) (end 157.8615 90.17) (width 0.25) (layer "F.Cu") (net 13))
 (segment (start 156.718 98.044) (end 156.718 104.3834) (width 0.25) (layer "F.Cu") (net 13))
 (segment (start 154.559 107.889) (end 154.559 108.364) (width 0.25) (layer "F.Cu") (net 13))
 (segment (start 149.298 102.964) (end 150.749 102.964) (width 0.25) (layer "F.Cu") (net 14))
 (segment (start 147.9727 93.3627) (end 147.9727 87.8486) (width 0.25) (layer "F.Cu") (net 14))
 (segment (start 149.098 85.598) (end 149.098 86.7233) (width 0.25) (layer "F.Cu") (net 14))
 (segment (start 159.512 101.092) (end 165.608 94.996) (width 0.25) (layer "F.Cu") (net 14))
 (segment (start 147.828 104.434) (end 149.298 102.964) (width 0.25) (layer "F.Cu") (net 14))
 (segment (start 147.9727 87.8486) (end 149.098 86.7233) (width 0.25) (layer "F.Cu") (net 14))
 (segment (start 149.098 94.488) (end 147.9727 93.3627) (width 0.25) (layer "F.Cu") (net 14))
 (segment (start 165.608 94.996) (end 165.608 92.71) (width 0.25) (layer "F.Cu") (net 14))
 (segment (start 162.306 103.886) (end 159.512 101.092) (width 0.25) (layer "B.Cu") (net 14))
 (segment (start 147.066 96.5841) (end 148.0245 95.6256) (width 0.25) (layer "B.Cu") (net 14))
 (segment (start 151.17 101.092) (end 150.845 101.417) (width 0.25) (layer "B.Cu") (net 14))
 (segment (start 147.066 98.806) (end 147.066 96.5841) (width 0.25) (layer "B.Cu") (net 14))
 (segment (start 148.0245 95.5615) (end 149.098 94.488) (width 0.25) (layer "B.Cu") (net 14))
 (segment (start 150.845 101.417) (end 147.828 104.434) (width 0.25) (layer "B.Cu") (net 14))
 (segment (start 148.0245 95.6256) (end 148.0245 95.5615) (width 0.25) (layer "B.Cu") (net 14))
 (segment (start 159.512 101.092) (end 151.17 101.092) (width 0.25) (layer "B.Cu") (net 14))
 (segment (start 150.261 102.001) (end 147.066 98.806) (width 0.25) (layer "B.Cu") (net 14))
 (segment (start 150.845 101.417) (end 150.261 102.001) (width 0.25) (layer "B.Cu") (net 14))
 (segment (start 165.608 120.494) (end 162.306 117.192) (width 0.25) (layer "B.Cu") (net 14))
 (segment (start 162.306 117.192) (end 162.306 103.886) (width 0.25) (layer "B.Cu") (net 14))
 (segment (start 154.559 102.964) (end 154.559 83.185) (width 0.25) (layer "F.Cu") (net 12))
 (segment (start 154.559 83.185) (end 156.718 81.026) (width 0.25) (layer "F.Cu") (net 12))
 (segment (start 136.652 94.488) (end 137.7773 94.488) (width 0.25) (layer "B.Cu") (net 12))
 (segment (start 144.3813 87.884) (end 137.7773 94.488) (width 0.25) (layer "B.Cu") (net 12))
 (segment (start 149.86 87.884) (end 144.3813 87.884) (width 0.25) (layer "B.Cu") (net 12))
 (segment (start 156.718 81.026) (end 149.86 87.884) (width 0.25) (layer "B.Cu") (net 12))
 (segment (start 165.608 113.03) (end 165.608 117.954) (width 0.25) (layer "F.Cu") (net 20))
 (segment (start 149.098 116.105) (end 149.098 114.9797) (width 0.25) (layer "F.Cu") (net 15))
 (segment (start 146.6928 100.4492) (end 146.6928 107.4046) (width 0.25) (layer "F.Cu") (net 15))
 (segment (start 149.098 98.044) (end 146.6928 100.4492) (width 0.25) (layer "F.Cu") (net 15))
 (segment (start 150.2233 110.9351) (end 150.2233 113.8544) (width 0.25) (layer "F.Cu") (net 15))
 (segment (start 150.2233 113.8544) (end 149.098 114.9797) (width 0.25) (layer "F.Cu") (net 15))
 (segment (start 146.6928 107.4046) (end 150.2233 110.9351) (width 0.25) (layer "F.Cu") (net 15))
 (segment (start 152.0367 98.044) (end 155.5927 94.488) (width 0.25) (layer "B.Cu") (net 15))
 (segment (start 156.718 94.488) (end 155.5927 94.488) (width 0.25) (layer "B.Cu") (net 15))
 (segment (start 149.098 98.044) (end 152.0367 98.044) (width 0.25) (layer "B.Cu") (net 15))
 (segment (start 153.2837 111.999) (end 156.718 111.999) (width 0.25) (layer "F.Cu") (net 16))
 (segment (start 150.749 109.4643) (end 153.2837 111.999) (width 0.25) (layer "F.Cu") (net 16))
 (segment (start 150.749 108.364) (end 150.749 109.4643) (width 0.25) (layer "F.Cu") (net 16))
 (segment (start 159.512 109.22) (end 158.8947 109.8373) (width 0.25) (layer "B.Cu") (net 16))
 (segment (start 158.8947 109.8373) (end 158.8797 109.8373) (width 0.25) (layer "B.Cu") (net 16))
 (segment (start 156.718 111.999) (end 158.8797 109.8373) (width 0.25) (layer "B.Cu") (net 16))
 (segment (start 159.512 108.712) (end 159.512 109.22) (width 0.25) (layer "B.Cu") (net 16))
 (segment (start 152.019 108.364) (end 152.019 109.389) (width 0.25) (layer "F.Cu") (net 17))
 (segment (start 158.242 114.581) (end 157.517999 115.305001) (width 0.25) (layer "F.Cu") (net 17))
 (segment (start 158.242 111.506) (end 158.242 114.581) (width 0.25) (layer "F.Cu") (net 17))
 (segment (start 149.098 119.6787) (end 152.6717 116.105) (width 0.25) (layer "F.Cu") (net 17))
 (segment (start 149.098 120.804) (end 149.098 119.6787) (width 0.25) (layer "F.Cu") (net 17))
 (segment (start 157.168011 110.432011) (end 158.242 111.506) (width 0.25) (layer "F.Cu") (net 17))
 (segment (start 152.019 109.389) (end 153.062011 110.432011) (width 0.25) (layer "F.Cu") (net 17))
 (segment (start 157.517999 115.305001) (end 156.718 116.105) (width 0.25) (layer "F.Cu") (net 17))
 (segment (start 153.062011 110.432011) (end 157.168011 110.432011) (width 0.25) (layer "F.Cu") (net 17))
 (segment (start 152.6717 116.105) (end 156.718 116.105) (width 0.25) (layer "F.Cu") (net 17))
 (segment (start 157.48 109.982) (end 154.432 109.982) (width 0.25) (layer "F.Cu") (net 18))
 (segment (start 165.608 105.41) (end 164.4827 105.41) (width 0.25) (layer "F.Cu") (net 18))
 (segment (start 159.258 118.264) (end 156.718 120.804) (width 0.25) (layer "F.Cu") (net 18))
 (segment (start 159.258 110.6347) (end 159.258 111.506) (width 0.25) (layer "F.Cu") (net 18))
 (segment (start 159.258 111.76) (end 159.258 118.264) (width 0.25) (layer "F.Cu") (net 18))
 (segment (start 159.258 111.506) (end 159.258 111.76) (width 0.25) (layer "F.Cu") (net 18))
 (segment (start 154.432 109.982) (end 153.289 108.839) (width 0.25) (layer "F.Cu") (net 18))
 (segment (start 153.289 108.839) (end 153.289 108.364) (width 0.25) (layer "F.Cu") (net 18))
 (segment (start 159.258 111.76) (end 157.48 109.982) (width 0.25) (layer "F.Cu") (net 18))
 (segment (start 164.4827 105.41) (end 159.258 110.6347) (width 0.25) (layer "F.Cu") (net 18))
 (segment (start 153.289 102.964) (end 153.289 95.4863) (width 0.25) (layer "F.Cu") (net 19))
 (segment (start 149.098 90.17) (end 149.098 91.2953) (width 0.25) (layer "F.Cu") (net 19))
 (segment (start 153.289 95.4863) (end 149.098 91.2953) (width 0.25) (layer "F.Cu") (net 19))
 (segment (start 154.7953 85.598) (end 156.718 85.598) (width 0.25) (layer "B.Cu") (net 19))
 (segment (start 149.098 90.17) (end 150.2233 90.17) (width 0.25) (layer "B.Cu") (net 19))
 (segment (start 150.2233 90.17) (end 154.7953 85.598) (width 0.25) (layer "B.Cu") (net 19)))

